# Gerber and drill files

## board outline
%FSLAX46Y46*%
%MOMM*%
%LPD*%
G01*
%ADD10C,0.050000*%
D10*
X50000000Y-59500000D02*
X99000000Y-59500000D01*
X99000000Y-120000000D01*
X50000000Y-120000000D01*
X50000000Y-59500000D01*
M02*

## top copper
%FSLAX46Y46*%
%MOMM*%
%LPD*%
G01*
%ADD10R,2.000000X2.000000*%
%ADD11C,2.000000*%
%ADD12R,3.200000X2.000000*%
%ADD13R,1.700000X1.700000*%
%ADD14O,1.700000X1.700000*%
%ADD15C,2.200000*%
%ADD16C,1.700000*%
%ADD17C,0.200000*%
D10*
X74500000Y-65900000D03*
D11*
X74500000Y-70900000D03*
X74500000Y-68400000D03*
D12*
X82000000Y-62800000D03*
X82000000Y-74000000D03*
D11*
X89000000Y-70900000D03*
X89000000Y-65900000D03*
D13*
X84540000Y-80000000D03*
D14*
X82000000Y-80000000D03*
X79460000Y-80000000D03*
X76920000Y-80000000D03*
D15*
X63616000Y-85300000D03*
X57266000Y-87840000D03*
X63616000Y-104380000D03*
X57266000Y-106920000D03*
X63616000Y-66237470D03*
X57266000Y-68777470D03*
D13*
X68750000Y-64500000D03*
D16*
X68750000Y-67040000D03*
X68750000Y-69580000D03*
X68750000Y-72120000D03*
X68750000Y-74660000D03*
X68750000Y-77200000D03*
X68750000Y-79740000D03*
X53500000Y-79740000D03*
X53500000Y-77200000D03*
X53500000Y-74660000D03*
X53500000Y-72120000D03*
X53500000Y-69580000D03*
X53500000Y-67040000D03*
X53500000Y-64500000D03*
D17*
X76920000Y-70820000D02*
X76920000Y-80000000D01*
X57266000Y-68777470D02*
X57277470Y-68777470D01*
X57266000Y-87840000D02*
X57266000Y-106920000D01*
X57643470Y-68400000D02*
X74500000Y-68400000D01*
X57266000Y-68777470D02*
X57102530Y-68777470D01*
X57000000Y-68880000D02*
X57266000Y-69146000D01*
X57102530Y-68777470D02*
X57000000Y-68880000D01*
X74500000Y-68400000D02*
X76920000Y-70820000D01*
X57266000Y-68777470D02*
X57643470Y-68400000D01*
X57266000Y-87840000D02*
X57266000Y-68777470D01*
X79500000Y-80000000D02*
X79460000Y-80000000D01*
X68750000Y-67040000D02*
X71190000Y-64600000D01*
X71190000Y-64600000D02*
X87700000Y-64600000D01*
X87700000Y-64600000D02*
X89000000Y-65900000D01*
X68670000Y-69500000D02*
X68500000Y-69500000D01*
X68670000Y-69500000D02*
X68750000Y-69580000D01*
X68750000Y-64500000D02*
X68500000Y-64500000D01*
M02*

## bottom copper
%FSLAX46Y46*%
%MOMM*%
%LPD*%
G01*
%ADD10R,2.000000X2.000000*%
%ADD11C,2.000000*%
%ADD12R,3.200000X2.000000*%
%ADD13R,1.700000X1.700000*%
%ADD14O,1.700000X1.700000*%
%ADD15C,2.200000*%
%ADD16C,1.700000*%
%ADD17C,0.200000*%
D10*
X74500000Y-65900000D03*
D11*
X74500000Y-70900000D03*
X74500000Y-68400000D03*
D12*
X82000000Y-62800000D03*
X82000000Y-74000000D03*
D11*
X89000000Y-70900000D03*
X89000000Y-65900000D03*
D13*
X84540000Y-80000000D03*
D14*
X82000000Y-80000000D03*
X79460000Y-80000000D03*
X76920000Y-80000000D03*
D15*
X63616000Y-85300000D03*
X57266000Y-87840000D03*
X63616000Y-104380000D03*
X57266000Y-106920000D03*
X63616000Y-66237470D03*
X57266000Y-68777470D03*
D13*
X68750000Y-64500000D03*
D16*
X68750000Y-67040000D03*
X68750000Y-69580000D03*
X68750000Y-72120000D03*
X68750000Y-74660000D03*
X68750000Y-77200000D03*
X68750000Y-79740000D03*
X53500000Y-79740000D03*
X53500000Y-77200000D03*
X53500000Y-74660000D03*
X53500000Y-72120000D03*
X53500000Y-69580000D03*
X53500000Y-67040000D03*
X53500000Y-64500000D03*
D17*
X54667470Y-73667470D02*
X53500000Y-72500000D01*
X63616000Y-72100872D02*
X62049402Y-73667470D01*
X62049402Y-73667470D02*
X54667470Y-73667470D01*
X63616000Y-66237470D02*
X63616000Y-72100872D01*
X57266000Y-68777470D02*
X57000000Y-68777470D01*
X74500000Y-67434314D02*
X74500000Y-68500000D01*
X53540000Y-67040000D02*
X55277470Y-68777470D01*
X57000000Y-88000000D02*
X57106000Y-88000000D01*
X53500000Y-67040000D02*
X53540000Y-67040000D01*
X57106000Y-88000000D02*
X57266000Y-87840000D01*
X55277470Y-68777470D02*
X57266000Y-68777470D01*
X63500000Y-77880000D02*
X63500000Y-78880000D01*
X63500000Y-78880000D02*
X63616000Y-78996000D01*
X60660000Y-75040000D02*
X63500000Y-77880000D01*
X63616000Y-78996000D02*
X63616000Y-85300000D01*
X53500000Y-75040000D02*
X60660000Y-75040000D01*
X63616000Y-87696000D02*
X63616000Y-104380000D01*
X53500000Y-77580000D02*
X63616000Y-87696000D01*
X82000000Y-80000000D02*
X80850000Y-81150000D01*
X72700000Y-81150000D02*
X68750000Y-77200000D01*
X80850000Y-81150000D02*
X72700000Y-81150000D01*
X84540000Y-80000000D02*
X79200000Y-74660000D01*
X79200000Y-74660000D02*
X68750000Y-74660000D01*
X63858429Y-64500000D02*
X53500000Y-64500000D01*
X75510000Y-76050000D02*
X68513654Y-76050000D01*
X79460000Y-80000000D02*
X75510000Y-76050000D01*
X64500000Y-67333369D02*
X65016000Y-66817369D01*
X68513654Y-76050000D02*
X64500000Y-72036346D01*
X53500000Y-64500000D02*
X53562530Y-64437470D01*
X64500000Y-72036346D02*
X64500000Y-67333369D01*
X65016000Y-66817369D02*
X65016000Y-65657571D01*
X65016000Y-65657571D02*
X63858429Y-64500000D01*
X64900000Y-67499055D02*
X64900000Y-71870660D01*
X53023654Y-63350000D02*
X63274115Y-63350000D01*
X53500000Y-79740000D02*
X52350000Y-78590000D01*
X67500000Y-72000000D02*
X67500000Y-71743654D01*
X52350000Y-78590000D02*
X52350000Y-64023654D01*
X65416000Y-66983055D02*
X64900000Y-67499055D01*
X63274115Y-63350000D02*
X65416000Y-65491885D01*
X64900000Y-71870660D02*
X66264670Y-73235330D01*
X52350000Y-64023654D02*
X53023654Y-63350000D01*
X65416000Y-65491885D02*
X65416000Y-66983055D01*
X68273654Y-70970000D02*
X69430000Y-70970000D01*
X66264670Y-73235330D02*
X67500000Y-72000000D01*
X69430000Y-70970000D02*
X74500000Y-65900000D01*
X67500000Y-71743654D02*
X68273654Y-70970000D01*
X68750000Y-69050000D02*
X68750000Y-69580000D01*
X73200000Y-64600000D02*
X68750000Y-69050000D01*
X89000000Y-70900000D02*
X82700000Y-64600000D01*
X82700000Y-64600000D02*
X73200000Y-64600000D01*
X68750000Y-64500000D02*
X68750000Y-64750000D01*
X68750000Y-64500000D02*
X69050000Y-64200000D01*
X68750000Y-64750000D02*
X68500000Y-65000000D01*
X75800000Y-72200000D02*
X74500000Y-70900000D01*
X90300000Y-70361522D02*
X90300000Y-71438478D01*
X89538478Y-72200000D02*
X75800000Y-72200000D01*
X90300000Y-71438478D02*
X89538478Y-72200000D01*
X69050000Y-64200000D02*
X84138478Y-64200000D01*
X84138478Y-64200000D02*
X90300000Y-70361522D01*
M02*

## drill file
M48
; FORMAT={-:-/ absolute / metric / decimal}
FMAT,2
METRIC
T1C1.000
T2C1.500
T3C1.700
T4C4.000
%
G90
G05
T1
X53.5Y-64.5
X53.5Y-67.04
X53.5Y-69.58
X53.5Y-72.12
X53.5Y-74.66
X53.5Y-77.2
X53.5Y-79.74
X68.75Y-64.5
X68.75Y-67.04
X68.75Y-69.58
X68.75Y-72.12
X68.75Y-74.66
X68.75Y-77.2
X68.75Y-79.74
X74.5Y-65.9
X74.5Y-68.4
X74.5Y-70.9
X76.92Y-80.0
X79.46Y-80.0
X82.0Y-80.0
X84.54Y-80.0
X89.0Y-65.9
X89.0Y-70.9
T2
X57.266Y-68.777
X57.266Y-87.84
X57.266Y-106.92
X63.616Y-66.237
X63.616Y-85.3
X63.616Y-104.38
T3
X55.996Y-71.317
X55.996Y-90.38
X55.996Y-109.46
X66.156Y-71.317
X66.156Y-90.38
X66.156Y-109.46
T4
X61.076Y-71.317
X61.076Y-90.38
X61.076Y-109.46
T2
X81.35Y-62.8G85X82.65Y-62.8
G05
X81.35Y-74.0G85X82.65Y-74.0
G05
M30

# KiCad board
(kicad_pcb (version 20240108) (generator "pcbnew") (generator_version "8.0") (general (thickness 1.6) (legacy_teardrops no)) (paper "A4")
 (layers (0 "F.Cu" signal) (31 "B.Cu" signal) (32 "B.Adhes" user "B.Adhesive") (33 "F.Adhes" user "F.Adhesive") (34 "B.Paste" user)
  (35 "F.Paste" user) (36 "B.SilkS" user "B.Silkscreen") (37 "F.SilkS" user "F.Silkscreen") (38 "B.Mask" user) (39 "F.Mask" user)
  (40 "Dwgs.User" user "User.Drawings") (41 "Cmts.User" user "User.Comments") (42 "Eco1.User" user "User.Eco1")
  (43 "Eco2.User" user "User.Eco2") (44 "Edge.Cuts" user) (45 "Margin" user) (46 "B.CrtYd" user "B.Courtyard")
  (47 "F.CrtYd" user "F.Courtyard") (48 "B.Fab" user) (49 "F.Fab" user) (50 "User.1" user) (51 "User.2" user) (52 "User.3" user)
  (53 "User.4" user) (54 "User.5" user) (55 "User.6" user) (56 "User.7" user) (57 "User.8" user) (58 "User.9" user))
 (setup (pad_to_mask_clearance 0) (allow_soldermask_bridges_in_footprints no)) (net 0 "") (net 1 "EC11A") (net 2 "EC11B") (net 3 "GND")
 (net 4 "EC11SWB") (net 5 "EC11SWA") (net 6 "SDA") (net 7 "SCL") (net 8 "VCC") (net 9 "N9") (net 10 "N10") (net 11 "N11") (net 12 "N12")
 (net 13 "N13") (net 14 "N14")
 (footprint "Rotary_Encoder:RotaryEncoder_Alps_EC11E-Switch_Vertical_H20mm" (layer "F.Cu") (at 74.5 65.9)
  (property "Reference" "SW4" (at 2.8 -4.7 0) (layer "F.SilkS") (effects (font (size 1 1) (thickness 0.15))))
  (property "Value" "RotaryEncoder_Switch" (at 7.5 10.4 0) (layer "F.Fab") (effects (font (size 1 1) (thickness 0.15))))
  (pad "A" thru_hole rect (at 0 0) (size 2 2) (drill 1) (layers "*.Cu" "*.Mask") (remove_unused_layers no) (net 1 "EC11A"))
  (pad "B" thru_hole circle (at 0 5) (size 2 2) (drill 1) (layers "*.Cu" "*.Mask") (remove_unused_layers no) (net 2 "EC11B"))
  (pad "C" thru_hole circle (at 0 2.5) (size 2 2) (drill 1) (layers "*.Cu" "*.Mask") (remove_unused_layers no) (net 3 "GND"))
  (pad "MP" thru_hole rect (at 7.5 -3.1) (size 3.2 2) (drill oval 2.8 1.5) (layers "*.Cu" "*.Mask") (remove_unused_layers no))
  (pad "MP" thru_hole rect (at 7.5 8.1) (size 3.2 2) (drill oval 2.8 1.5) (layers "*.Cu" "*.Mask") (remove_unused_layers no))
  (pad "S1" thru_hole circle (at 14.5 5) (size 2 2) (drill 1) (layers "*.Cu" "*.Mask") (remove_unused_layers no) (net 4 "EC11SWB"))
  (pad "S2" thru_hole circle (at 14.5 0) (size 2 2) (drill 1) (layers "*.Cu" "*.Mask") (remove_unused_layers no) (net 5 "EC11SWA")))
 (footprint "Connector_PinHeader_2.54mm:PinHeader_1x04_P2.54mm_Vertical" (layer "F.Cu") (at 84.54 80 -90)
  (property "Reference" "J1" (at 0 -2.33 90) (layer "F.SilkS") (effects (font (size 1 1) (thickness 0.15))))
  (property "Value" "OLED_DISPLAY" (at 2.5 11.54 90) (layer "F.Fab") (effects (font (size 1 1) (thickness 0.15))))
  (pad "1" thru_hole rect (at 0 0 270) (size 1.7 1.7) (drill 1) (layers "*.Cu" "*.Mask") (remove_unused_layers no) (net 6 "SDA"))
  (pad "2" thru_hole oval (at 0 2.54 270) (size 1.7 1.7) (drill 1) (layers "*.Cu" "*.Mask") (remove_unused_layers no) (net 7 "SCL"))
  (pad "3" thru_hole oval (at 0 5.08 270) (size 1.7 1.7) (drill 1) (layers "*.Cu" "*.Mask") (remove_unused_layers no) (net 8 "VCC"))
  (pad "4" thru_hole oval (at 0 7.62 270) (size 1.7 1.7) (drill 1) (layers "*.Cu" "*.Mask") (remove_unused_layers no) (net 3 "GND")))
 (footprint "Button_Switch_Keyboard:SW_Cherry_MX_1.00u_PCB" (layer "F.Cu") (at 63.616 85.3)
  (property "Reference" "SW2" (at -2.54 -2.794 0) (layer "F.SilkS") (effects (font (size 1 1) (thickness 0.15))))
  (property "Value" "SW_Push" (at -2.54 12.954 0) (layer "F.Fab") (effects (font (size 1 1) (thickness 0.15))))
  (pad "" np_thru_hole circle (at -7.62 5.08) (size 1.7 1.7) (drill 1.7) (layers "*.Cu" "*.Mask"))
  (pad "" np_thru_hole circle (at -2.54 5.08) (size 4 4) (drill 4) (layers "*.Cu" "*.Mask"))
  (pad "" np_thru_hole circle (at 2.54 5.08) (size 1.7 1.7) (drill 1.7) (layers "*.Cu" "*.Mask"))
  (pad "1" thru_hole circle (at 0 0) (size 2.2 2.2) (drill 1.5) (layers "*.Cu" "*.Mask") (remove_unused_layers no) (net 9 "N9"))
  (pad "2" thru_hole circle (at -6.35 2.54) (size 2.2 2.2) (drill 1.5) (layers "*.Cu" "*.Mask") (remove_unused_layers no) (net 3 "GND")))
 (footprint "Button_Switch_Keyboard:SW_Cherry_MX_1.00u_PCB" (layer "F.Cu") (at 63.616 104.38)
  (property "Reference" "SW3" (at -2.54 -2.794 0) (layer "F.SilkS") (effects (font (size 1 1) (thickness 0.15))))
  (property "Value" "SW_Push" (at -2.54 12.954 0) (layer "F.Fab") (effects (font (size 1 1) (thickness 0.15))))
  (pad "" np_thru_hole circle (at -7.62 5.08) (size 1.7 1.7) (drill 1.7) (layers "*.Cu" "*.Mask"))
  (pad "" np_thru_hole circle (at -2.54 5.08) (size 4 4) (drill 4) (layers "*.Cu" "*.Mask"))
  (pad "" np_thru_hole circle (at 2.54 5.08) (size 1.7 1.7) (drill 1.7) (layers "*.Cu" "*.Mask"))
  (pad "1" thru_hole circle (at 0 0) (size 2.2 2.2) (drill 1.5) (layers "*.Cu" "*.Mask") (remove_unused_layers no) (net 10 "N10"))
  (pad "2" thru_hole circle (at -6.35 2.54) (size 2.2 2.2) (drill 1.5) (layers "*.Cu" "*.Mask") (remove_unused_layers no) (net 3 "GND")))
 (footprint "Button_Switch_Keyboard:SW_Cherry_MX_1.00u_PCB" (layer "F.Cu") (at 63.616 66.23747)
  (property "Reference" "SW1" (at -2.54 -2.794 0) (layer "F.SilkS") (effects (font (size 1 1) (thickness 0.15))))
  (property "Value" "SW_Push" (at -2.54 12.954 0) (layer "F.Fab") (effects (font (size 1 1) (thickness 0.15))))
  (pad "" np_thru_hole circle (at -7.62 5.08) (size 1.7 1.7) (drill 1.7) (layers "*.Cu" "*.Mask"))
  (pad "" np_thru_hole circle (at -2.54 5.08) (size 4 4) (drill 4) (layers "*.Cu" "*.Mask"))
  (pad "" np_thru_hole circle (at 2.54 5.08) (size 1.7 1.7) (drill 1.7) (layers "*.Cu" "*.Mask"))
  (pad "1" thru_hole circle (at 0 0) (size 2.2 2.2) (drill 1.5) (layers "*.Cu" "*.Mask") (remove_unused_layers no) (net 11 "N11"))
  (pad "2" thru_hole circle (at -6.35 2.54) (size 2.2 2.2) (drill 1.5) (layers "*.Cu" "*.Mask") (remove_unused_layers no) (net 3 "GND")))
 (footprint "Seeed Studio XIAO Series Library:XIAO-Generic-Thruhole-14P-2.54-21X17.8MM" (layer "B.Cu") (at 61.125 72.12 180)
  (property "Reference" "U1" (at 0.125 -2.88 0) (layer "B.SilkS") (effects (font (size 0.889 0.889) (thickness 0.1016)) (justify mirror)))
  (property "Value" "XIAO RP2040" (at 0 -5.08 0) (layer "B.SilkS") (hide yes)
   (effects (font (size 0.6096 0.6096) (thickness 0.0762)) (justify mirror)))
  (pad "1" thru_hole rect (at -7.625 7.62 180) (size 1.7 1.7) (drill 1) (layers "*.Cu" "*.Mask") (remove_unused_layers no) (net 2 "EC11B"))
  (pad "2" thru_hole circle (at -7.625 5.08 180) (size 1.7 1.7) (drill 1) (layers "*.Cu" "*.Mask") (remove_unused_layers no)
   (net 5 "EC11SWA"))
  (pad "3" thru_hole circle (at -7.625 2.54 180) (size 1.7 1.7) (drill 1) (layers "*.Cu" "*.Mask") (remove_unused_layers no)
   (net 4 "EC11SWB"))
  (pad "4" thru_hole circle (at -7.625 0 180) (size 1.7 1.7) (drill 1) (layers "*.Cu" "*.Mask") (remove_unused_layers no) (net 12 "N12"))
  (pad "5" thru_hole circle (at -7.625 -2.54 180) (size 1.7 1.7) (drill 1) (layers "*.Cu" "*.Mask") (remove_unused_layers no) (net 6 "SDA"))
  (pad "6" thru_hole circle (at -7.625 -5.08) (size 1.7 1.7) (drill 1) (layers "*.Cu" "*.Mask") (remove_unused_layers no) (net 7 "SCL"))
  (pad "7" thru_hole circle (at -7.625 -7.62 180) (size 1.7 1.7) (drill 1) (layers "*.Cu" "*.Mask") (remove_unused_layers no) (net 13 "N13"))
  (pad "8" thru_hole circle (at 7.625 -7.62 180) (size 1.7 1.7) (drill 1) (layers "*.Cu" "*.Mask") (remove_unused_layers no) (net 1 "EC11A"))
  (pad "9" thru_hole circle (at 7.625 -5.08 180) (size 1.7 1.7) (drill 1) (layers "*.Cu" "*.Mask") (remove_unused_layers no) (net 10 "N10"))
  (pad "10" thru_hole circle (at 7.625 -2.54 180) (size 1.7 1.7) (drill 1) (layers "*.Cu" "*.Mask") (remove_unused_layers no) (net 9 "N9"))
  (pad "11" thru_hole circle (at 7.625 0 180) (size 1.7 1.7) (drill 1) (layers "*.Cu" "*.Mask") (remove_unused_layers no) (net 11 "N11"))
  (pad "12" thru_hole circle (at 7.625 2.54 180) (size 1.7 1.7) (drill 1) (layers "*.Cu" "*.Mask") (remove_unused_layers no) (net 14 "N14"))
  (pad "13" thru_hole circle (at 7.625 5.08 180) (size 1.7 1.7) (drill 1) (layers "*.Cu" "*.Mask") (remove_unused_layers no) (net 3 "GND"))
  (pad "14" thru_hole circle (at 7.625 7.62 180) (size 1.7 1.7) (drill 1) (layers "*.Cu" "*.Mask") (remove_unused_layers no) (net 8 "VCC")))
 (gr_rect (start 50 59.5) (end 99 120) (stroke (width 0.05) (type default)) (fill none) (layer "Edge.Cuts"))
 (segment (start 54.66747 73.66747) (end 53.5 72.5) (width 0.2) (layer "B.Cu") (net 11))
 (segment (start 63.616 72.100872) (end 62.049402 73.66747) (width 0.2) (layer "B.Cu") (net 11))
 (segment (start 62.049402 73.66747) (end 54.66747 73.66747) (width 0.2) (layer "B.Cu") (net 11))
 (segment (start 63.616 66.23747) (end 63.616 72.100872) (width 0.2) (layer "B.Cu") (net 11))
 (segment (start 76.92 70.82) (end 76.92 80) (width 0.2) (layer "F.Cu") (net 3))
 (segment (start 57.266 68.77747) (end 57.27747 68.77747) (width 0.2) (layer "F.Cu") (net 3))
 (segment (start 57.266 87.84) (end 57.266 106.92) (width 0.2) (layer "F.Cu") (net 3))
 (segment (start 57.64347 68.4) (end 74.5 68.4) (width 0.2) (layer "F.Cu") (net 3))
 (segment (start 57.266 68.77747) (end 57.10253 68.77747) (width 0.2) (layer "F.Cu") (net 3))
 (segment (start 57 68.88) (end 57.266 69.146) (width 0.2) (layer "F.Cu") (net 3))
 (segment (start 57.10253 68.77747) (end 57 68.88) (width 0.2) (layer "F.Cu") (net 3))
 (segment (start 74.5 68.4) (end 76.92 70.82) (width 0.2) (layer "F.Cu") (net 3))
 (segment (start 57.266 68.77747) (end 57.64347 68.4) (width 0.2) (layer "F.Cu") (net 3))
 (segment (start 57.266 87.84) (end 57.266 68.77747) (width 0.2) (layer "F.Cu") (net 3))
 (segment (start 57.266 68.77747) (end 57 68.77747) (width 0.2) (layer "B.Cu") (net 3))
 (segment (start 74.5 67.434314) (end 74.5 68.5) (width 0.2) (layer "B.Cu") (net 3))
 (segment (start 53.54 67.04) (end 55.27747 68.77747) (width 0.2) (layer "B.Cu") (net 3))
 (segment (start 57 88) (end 57.106 88) (width 0.2) (layer "B.Cu") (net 3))
 (segment (start 53.5 67.04) (end 53.54 67.04) (width 0.2) (layer "B.Cu") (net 3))
 (segment (start 57.106 88) (end 57.266 87.84) (width 0.2) (layer "B.Cu") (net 3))
 (segment (start 55.27747 68.77747) (end 57.266 68.77747) (width 0.2) (layer "B.Cu") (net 3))
 (segment (start 63.5 77.88) (end 63.5 78.88) (width 0.2) (layer "B.Cu") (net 9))
 (segment (start 63.5 78.88) (end 63.616 78.996) (width 0.2) (layer "B.Cu") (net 9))
 (segment (start 60.66 75.04) (end 63.5 77.88) (width 0.2) (layer "B.Cu") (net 9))
 (segment (start 63.616 78.996) (end 63.616 85.3) (width 0.2) (layer "B.Cu") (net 9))
 (segment (start 53.5 75.04) (end 60.66 75.04) (width 0.2) (layer "B.Cu") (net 9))
 (segment (start 63.616 87.696) (end 63.616 104.38) (width 0.2) (layer "B.Cu") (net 10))
 (segment (start 53.5 77.58) (end 63.616 87.696) (width 0.2) (layer "B.Cu") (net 10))
 (segment (start 82 80) (end 80.85 81.15) (width 0.2) (layer "B.Cu") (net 7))
 (segment (start 72.7 81.15) (end 68.75 77.2) (width 0.2) (layer "B.Cu") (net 7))
 (segment (start 80.85 81.15) (end 72.7 81.15) (width 0.2) (layer "B.Cu") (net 7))
 (segment (start 84.54 80) (end 79.2 74.66) (width 0.2) (layer "B.Cu") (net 6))
 (segment (start 79.2 74.66) (end 68.75 74.66) (width 0.2) (layer "B.Cu") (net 6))
 (segment (start 79.5 80) (end 79.46 80) (width 0.2) (layer "F.Cu") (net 8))
 (segment (start 63.858429 64.5) (end 53.5 64.5) (width 0.2) (layer "B.Cu") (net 8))
 (segment (start 75.51 76.05) (end 68.513654 76.05) (width 0.2) (layer "B.Cu") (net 8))
 (segment (start 79.46 80) (end 75.51 76.05) (width 0.2) (layer "B.Cu") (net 8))
 (segment (start 64.5 67.333369) (end 65.016 66.817369) (width 0.2) (layer "B.Cu") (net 8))
 (segment (start 68.513654 76.05) (end 64.5 72.036346) (width 0.2) (layer "B.Cu") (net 8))
 (segment (start 53.5 64.5) (end 53.56253 64.43747) (width 0.2) (layer "B.Cu") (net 8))
 (segment (start 64.5 72.036346) (end 64.5 67.333369) (width 0.2) (layer "B.Cu") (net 8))
 (segment (start 65.016 66.817369) (end 65.016 65.657571) (width 0.2) (layer "B.Cu") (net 8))
 (segment (start 65.016 65.657571) (end 63.858429 64.5) (width 0.2) (layer "B.Cu") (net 8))
 (segment (start 68.75 67.04) (end 71.19 64.6) (width 0.2) (layer "F.Cu") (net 5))
 (segment (start 71.19 64.6) (end 87.7 64.6) (width 0.2) (layer "F.Cu") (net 5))
 (segment (start 87.7 64.6) (end 89 65.9) (width 0.2) (layer "F.Cu") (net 5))
 (segment (start 64.9 67.499055) (end 64.9 71.87066) (width 0.2) (layer "B.Cu") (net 1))
 (segment (start 53.023654 63.35) (end 63.274115 63.35) (width 0.2) (layer "B.Cu") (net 1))
 (segment (start 53.5 79.74) (end 52.35 78.59) (width 0.2) (layer "B.Cu") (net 1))
 (segment (start 67.5 72) (end 67.5 71.743654) (width 0.2) (layer "B.Cu") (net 1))
 (segment (start 52.35 78.59) (end 52.35 64.023654) (width 0.2) (layer "B.Cu") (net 1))
 (segment (start 65.416 66.983055) (end 64.9 67.499055) (width 0.2) (layer "B.Cu") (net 1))
 (segment (start 63.274115 63.35) (end 65.416 65.491885) (width 0.2) (layer "B.Cu") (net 1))
 (segment (start 64.9 71.87066) (end 66.26467 73.23533) (width 0.2) (layer "B.Cu") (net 1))
 (segment (start 52.35 64.023654) (end 53.023654 63.35) (width 0.2) (layer "B.Cu") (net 1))
 (segment (start 65.416 65.491885) (end 65.416 66.983055) (width 0.2) (layer "B.Cu") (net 1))
 (segment (start 68.273654 70.97) (end 69.43 70.97) (width 0.2) (layer "B.Cu") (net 1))
 (segment (start 66.26467 73.23533) (end 67.5 72) (width 0.2) (layer "B.Cu") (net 1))
 (segment (start 69.43 70.97) (end 74.5 65.9) (width 0.2) (layer "B.Cu") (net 1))
 (segment (start 67.5 71.743654) (end 68.273654 70.97) (width 0.2) (layer "B.Cu") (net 1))
 (segment (start 68.67 69.5) (end 68.5 69.5) (width 0.2) (layer "F.Cu") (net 4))
 (segment (start 68.67 69.5) (end 68.75 69.58) (width 0.2) (layer "F.Cu") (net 4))
 (segment (start 68.75 69.05) (end 68.75 69.58) (width 0.2) (layer "B.Cu") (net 4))
 (segment (start 73.2 64.6) (end 68.75 69.05) (width 0.2) (layer "B.Cu") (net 4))
 (segment (start 89 70.9) (end 82.7 64.6) (width 0.2) (layer "B.Cu") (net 4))
 (segment (start 82.7 64.6) (end 73.2 64.6) (width 0.2) (layer "B.Cu") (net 4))
 (segment (start 68.75 64.5) (end 68.5 64.5) (width 0.2) (layer "F.Cu") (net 2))
 (segment (start 68.75 64.5) (end 68.75 64.75) (width 0.2) (layer "B.Cu") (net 2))
 (segment (start 68.75 64.5) (end 69.05 64.2) (width 0.2) (layer "B.Cu") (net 2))
 (segment (start 68.75 64.75) (end 68.5 65) (width 0.2) (layer "B.Cu") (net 2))
 (segment (start 75.8 72.2) (end 74.5 70.9) (width 0.2) (layer "B.Cu") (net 2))
 (segment (start 90.3 70.361522) (end 90.3 71.438478) (width 0.2) (layer "B.Cu") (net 2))
 (segment (start 89.538478 72.2) (end 75.8 72.2) (width 0.2) (layer "B.Cu") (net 2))
 (segment (start 90.3 71.438478) (end 89.538478 72.2) (width 0.2) (layer "B.Cu") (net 2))
 (segment (start 69.05 64.2) (end 84.138478 64.2) (width 0.2) (layer "B.Cu") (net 2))
 (segment (start 84.138478 64.2) (end 90.3 70.361522) (width 0.2) (layer "B.Cu") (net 2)))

